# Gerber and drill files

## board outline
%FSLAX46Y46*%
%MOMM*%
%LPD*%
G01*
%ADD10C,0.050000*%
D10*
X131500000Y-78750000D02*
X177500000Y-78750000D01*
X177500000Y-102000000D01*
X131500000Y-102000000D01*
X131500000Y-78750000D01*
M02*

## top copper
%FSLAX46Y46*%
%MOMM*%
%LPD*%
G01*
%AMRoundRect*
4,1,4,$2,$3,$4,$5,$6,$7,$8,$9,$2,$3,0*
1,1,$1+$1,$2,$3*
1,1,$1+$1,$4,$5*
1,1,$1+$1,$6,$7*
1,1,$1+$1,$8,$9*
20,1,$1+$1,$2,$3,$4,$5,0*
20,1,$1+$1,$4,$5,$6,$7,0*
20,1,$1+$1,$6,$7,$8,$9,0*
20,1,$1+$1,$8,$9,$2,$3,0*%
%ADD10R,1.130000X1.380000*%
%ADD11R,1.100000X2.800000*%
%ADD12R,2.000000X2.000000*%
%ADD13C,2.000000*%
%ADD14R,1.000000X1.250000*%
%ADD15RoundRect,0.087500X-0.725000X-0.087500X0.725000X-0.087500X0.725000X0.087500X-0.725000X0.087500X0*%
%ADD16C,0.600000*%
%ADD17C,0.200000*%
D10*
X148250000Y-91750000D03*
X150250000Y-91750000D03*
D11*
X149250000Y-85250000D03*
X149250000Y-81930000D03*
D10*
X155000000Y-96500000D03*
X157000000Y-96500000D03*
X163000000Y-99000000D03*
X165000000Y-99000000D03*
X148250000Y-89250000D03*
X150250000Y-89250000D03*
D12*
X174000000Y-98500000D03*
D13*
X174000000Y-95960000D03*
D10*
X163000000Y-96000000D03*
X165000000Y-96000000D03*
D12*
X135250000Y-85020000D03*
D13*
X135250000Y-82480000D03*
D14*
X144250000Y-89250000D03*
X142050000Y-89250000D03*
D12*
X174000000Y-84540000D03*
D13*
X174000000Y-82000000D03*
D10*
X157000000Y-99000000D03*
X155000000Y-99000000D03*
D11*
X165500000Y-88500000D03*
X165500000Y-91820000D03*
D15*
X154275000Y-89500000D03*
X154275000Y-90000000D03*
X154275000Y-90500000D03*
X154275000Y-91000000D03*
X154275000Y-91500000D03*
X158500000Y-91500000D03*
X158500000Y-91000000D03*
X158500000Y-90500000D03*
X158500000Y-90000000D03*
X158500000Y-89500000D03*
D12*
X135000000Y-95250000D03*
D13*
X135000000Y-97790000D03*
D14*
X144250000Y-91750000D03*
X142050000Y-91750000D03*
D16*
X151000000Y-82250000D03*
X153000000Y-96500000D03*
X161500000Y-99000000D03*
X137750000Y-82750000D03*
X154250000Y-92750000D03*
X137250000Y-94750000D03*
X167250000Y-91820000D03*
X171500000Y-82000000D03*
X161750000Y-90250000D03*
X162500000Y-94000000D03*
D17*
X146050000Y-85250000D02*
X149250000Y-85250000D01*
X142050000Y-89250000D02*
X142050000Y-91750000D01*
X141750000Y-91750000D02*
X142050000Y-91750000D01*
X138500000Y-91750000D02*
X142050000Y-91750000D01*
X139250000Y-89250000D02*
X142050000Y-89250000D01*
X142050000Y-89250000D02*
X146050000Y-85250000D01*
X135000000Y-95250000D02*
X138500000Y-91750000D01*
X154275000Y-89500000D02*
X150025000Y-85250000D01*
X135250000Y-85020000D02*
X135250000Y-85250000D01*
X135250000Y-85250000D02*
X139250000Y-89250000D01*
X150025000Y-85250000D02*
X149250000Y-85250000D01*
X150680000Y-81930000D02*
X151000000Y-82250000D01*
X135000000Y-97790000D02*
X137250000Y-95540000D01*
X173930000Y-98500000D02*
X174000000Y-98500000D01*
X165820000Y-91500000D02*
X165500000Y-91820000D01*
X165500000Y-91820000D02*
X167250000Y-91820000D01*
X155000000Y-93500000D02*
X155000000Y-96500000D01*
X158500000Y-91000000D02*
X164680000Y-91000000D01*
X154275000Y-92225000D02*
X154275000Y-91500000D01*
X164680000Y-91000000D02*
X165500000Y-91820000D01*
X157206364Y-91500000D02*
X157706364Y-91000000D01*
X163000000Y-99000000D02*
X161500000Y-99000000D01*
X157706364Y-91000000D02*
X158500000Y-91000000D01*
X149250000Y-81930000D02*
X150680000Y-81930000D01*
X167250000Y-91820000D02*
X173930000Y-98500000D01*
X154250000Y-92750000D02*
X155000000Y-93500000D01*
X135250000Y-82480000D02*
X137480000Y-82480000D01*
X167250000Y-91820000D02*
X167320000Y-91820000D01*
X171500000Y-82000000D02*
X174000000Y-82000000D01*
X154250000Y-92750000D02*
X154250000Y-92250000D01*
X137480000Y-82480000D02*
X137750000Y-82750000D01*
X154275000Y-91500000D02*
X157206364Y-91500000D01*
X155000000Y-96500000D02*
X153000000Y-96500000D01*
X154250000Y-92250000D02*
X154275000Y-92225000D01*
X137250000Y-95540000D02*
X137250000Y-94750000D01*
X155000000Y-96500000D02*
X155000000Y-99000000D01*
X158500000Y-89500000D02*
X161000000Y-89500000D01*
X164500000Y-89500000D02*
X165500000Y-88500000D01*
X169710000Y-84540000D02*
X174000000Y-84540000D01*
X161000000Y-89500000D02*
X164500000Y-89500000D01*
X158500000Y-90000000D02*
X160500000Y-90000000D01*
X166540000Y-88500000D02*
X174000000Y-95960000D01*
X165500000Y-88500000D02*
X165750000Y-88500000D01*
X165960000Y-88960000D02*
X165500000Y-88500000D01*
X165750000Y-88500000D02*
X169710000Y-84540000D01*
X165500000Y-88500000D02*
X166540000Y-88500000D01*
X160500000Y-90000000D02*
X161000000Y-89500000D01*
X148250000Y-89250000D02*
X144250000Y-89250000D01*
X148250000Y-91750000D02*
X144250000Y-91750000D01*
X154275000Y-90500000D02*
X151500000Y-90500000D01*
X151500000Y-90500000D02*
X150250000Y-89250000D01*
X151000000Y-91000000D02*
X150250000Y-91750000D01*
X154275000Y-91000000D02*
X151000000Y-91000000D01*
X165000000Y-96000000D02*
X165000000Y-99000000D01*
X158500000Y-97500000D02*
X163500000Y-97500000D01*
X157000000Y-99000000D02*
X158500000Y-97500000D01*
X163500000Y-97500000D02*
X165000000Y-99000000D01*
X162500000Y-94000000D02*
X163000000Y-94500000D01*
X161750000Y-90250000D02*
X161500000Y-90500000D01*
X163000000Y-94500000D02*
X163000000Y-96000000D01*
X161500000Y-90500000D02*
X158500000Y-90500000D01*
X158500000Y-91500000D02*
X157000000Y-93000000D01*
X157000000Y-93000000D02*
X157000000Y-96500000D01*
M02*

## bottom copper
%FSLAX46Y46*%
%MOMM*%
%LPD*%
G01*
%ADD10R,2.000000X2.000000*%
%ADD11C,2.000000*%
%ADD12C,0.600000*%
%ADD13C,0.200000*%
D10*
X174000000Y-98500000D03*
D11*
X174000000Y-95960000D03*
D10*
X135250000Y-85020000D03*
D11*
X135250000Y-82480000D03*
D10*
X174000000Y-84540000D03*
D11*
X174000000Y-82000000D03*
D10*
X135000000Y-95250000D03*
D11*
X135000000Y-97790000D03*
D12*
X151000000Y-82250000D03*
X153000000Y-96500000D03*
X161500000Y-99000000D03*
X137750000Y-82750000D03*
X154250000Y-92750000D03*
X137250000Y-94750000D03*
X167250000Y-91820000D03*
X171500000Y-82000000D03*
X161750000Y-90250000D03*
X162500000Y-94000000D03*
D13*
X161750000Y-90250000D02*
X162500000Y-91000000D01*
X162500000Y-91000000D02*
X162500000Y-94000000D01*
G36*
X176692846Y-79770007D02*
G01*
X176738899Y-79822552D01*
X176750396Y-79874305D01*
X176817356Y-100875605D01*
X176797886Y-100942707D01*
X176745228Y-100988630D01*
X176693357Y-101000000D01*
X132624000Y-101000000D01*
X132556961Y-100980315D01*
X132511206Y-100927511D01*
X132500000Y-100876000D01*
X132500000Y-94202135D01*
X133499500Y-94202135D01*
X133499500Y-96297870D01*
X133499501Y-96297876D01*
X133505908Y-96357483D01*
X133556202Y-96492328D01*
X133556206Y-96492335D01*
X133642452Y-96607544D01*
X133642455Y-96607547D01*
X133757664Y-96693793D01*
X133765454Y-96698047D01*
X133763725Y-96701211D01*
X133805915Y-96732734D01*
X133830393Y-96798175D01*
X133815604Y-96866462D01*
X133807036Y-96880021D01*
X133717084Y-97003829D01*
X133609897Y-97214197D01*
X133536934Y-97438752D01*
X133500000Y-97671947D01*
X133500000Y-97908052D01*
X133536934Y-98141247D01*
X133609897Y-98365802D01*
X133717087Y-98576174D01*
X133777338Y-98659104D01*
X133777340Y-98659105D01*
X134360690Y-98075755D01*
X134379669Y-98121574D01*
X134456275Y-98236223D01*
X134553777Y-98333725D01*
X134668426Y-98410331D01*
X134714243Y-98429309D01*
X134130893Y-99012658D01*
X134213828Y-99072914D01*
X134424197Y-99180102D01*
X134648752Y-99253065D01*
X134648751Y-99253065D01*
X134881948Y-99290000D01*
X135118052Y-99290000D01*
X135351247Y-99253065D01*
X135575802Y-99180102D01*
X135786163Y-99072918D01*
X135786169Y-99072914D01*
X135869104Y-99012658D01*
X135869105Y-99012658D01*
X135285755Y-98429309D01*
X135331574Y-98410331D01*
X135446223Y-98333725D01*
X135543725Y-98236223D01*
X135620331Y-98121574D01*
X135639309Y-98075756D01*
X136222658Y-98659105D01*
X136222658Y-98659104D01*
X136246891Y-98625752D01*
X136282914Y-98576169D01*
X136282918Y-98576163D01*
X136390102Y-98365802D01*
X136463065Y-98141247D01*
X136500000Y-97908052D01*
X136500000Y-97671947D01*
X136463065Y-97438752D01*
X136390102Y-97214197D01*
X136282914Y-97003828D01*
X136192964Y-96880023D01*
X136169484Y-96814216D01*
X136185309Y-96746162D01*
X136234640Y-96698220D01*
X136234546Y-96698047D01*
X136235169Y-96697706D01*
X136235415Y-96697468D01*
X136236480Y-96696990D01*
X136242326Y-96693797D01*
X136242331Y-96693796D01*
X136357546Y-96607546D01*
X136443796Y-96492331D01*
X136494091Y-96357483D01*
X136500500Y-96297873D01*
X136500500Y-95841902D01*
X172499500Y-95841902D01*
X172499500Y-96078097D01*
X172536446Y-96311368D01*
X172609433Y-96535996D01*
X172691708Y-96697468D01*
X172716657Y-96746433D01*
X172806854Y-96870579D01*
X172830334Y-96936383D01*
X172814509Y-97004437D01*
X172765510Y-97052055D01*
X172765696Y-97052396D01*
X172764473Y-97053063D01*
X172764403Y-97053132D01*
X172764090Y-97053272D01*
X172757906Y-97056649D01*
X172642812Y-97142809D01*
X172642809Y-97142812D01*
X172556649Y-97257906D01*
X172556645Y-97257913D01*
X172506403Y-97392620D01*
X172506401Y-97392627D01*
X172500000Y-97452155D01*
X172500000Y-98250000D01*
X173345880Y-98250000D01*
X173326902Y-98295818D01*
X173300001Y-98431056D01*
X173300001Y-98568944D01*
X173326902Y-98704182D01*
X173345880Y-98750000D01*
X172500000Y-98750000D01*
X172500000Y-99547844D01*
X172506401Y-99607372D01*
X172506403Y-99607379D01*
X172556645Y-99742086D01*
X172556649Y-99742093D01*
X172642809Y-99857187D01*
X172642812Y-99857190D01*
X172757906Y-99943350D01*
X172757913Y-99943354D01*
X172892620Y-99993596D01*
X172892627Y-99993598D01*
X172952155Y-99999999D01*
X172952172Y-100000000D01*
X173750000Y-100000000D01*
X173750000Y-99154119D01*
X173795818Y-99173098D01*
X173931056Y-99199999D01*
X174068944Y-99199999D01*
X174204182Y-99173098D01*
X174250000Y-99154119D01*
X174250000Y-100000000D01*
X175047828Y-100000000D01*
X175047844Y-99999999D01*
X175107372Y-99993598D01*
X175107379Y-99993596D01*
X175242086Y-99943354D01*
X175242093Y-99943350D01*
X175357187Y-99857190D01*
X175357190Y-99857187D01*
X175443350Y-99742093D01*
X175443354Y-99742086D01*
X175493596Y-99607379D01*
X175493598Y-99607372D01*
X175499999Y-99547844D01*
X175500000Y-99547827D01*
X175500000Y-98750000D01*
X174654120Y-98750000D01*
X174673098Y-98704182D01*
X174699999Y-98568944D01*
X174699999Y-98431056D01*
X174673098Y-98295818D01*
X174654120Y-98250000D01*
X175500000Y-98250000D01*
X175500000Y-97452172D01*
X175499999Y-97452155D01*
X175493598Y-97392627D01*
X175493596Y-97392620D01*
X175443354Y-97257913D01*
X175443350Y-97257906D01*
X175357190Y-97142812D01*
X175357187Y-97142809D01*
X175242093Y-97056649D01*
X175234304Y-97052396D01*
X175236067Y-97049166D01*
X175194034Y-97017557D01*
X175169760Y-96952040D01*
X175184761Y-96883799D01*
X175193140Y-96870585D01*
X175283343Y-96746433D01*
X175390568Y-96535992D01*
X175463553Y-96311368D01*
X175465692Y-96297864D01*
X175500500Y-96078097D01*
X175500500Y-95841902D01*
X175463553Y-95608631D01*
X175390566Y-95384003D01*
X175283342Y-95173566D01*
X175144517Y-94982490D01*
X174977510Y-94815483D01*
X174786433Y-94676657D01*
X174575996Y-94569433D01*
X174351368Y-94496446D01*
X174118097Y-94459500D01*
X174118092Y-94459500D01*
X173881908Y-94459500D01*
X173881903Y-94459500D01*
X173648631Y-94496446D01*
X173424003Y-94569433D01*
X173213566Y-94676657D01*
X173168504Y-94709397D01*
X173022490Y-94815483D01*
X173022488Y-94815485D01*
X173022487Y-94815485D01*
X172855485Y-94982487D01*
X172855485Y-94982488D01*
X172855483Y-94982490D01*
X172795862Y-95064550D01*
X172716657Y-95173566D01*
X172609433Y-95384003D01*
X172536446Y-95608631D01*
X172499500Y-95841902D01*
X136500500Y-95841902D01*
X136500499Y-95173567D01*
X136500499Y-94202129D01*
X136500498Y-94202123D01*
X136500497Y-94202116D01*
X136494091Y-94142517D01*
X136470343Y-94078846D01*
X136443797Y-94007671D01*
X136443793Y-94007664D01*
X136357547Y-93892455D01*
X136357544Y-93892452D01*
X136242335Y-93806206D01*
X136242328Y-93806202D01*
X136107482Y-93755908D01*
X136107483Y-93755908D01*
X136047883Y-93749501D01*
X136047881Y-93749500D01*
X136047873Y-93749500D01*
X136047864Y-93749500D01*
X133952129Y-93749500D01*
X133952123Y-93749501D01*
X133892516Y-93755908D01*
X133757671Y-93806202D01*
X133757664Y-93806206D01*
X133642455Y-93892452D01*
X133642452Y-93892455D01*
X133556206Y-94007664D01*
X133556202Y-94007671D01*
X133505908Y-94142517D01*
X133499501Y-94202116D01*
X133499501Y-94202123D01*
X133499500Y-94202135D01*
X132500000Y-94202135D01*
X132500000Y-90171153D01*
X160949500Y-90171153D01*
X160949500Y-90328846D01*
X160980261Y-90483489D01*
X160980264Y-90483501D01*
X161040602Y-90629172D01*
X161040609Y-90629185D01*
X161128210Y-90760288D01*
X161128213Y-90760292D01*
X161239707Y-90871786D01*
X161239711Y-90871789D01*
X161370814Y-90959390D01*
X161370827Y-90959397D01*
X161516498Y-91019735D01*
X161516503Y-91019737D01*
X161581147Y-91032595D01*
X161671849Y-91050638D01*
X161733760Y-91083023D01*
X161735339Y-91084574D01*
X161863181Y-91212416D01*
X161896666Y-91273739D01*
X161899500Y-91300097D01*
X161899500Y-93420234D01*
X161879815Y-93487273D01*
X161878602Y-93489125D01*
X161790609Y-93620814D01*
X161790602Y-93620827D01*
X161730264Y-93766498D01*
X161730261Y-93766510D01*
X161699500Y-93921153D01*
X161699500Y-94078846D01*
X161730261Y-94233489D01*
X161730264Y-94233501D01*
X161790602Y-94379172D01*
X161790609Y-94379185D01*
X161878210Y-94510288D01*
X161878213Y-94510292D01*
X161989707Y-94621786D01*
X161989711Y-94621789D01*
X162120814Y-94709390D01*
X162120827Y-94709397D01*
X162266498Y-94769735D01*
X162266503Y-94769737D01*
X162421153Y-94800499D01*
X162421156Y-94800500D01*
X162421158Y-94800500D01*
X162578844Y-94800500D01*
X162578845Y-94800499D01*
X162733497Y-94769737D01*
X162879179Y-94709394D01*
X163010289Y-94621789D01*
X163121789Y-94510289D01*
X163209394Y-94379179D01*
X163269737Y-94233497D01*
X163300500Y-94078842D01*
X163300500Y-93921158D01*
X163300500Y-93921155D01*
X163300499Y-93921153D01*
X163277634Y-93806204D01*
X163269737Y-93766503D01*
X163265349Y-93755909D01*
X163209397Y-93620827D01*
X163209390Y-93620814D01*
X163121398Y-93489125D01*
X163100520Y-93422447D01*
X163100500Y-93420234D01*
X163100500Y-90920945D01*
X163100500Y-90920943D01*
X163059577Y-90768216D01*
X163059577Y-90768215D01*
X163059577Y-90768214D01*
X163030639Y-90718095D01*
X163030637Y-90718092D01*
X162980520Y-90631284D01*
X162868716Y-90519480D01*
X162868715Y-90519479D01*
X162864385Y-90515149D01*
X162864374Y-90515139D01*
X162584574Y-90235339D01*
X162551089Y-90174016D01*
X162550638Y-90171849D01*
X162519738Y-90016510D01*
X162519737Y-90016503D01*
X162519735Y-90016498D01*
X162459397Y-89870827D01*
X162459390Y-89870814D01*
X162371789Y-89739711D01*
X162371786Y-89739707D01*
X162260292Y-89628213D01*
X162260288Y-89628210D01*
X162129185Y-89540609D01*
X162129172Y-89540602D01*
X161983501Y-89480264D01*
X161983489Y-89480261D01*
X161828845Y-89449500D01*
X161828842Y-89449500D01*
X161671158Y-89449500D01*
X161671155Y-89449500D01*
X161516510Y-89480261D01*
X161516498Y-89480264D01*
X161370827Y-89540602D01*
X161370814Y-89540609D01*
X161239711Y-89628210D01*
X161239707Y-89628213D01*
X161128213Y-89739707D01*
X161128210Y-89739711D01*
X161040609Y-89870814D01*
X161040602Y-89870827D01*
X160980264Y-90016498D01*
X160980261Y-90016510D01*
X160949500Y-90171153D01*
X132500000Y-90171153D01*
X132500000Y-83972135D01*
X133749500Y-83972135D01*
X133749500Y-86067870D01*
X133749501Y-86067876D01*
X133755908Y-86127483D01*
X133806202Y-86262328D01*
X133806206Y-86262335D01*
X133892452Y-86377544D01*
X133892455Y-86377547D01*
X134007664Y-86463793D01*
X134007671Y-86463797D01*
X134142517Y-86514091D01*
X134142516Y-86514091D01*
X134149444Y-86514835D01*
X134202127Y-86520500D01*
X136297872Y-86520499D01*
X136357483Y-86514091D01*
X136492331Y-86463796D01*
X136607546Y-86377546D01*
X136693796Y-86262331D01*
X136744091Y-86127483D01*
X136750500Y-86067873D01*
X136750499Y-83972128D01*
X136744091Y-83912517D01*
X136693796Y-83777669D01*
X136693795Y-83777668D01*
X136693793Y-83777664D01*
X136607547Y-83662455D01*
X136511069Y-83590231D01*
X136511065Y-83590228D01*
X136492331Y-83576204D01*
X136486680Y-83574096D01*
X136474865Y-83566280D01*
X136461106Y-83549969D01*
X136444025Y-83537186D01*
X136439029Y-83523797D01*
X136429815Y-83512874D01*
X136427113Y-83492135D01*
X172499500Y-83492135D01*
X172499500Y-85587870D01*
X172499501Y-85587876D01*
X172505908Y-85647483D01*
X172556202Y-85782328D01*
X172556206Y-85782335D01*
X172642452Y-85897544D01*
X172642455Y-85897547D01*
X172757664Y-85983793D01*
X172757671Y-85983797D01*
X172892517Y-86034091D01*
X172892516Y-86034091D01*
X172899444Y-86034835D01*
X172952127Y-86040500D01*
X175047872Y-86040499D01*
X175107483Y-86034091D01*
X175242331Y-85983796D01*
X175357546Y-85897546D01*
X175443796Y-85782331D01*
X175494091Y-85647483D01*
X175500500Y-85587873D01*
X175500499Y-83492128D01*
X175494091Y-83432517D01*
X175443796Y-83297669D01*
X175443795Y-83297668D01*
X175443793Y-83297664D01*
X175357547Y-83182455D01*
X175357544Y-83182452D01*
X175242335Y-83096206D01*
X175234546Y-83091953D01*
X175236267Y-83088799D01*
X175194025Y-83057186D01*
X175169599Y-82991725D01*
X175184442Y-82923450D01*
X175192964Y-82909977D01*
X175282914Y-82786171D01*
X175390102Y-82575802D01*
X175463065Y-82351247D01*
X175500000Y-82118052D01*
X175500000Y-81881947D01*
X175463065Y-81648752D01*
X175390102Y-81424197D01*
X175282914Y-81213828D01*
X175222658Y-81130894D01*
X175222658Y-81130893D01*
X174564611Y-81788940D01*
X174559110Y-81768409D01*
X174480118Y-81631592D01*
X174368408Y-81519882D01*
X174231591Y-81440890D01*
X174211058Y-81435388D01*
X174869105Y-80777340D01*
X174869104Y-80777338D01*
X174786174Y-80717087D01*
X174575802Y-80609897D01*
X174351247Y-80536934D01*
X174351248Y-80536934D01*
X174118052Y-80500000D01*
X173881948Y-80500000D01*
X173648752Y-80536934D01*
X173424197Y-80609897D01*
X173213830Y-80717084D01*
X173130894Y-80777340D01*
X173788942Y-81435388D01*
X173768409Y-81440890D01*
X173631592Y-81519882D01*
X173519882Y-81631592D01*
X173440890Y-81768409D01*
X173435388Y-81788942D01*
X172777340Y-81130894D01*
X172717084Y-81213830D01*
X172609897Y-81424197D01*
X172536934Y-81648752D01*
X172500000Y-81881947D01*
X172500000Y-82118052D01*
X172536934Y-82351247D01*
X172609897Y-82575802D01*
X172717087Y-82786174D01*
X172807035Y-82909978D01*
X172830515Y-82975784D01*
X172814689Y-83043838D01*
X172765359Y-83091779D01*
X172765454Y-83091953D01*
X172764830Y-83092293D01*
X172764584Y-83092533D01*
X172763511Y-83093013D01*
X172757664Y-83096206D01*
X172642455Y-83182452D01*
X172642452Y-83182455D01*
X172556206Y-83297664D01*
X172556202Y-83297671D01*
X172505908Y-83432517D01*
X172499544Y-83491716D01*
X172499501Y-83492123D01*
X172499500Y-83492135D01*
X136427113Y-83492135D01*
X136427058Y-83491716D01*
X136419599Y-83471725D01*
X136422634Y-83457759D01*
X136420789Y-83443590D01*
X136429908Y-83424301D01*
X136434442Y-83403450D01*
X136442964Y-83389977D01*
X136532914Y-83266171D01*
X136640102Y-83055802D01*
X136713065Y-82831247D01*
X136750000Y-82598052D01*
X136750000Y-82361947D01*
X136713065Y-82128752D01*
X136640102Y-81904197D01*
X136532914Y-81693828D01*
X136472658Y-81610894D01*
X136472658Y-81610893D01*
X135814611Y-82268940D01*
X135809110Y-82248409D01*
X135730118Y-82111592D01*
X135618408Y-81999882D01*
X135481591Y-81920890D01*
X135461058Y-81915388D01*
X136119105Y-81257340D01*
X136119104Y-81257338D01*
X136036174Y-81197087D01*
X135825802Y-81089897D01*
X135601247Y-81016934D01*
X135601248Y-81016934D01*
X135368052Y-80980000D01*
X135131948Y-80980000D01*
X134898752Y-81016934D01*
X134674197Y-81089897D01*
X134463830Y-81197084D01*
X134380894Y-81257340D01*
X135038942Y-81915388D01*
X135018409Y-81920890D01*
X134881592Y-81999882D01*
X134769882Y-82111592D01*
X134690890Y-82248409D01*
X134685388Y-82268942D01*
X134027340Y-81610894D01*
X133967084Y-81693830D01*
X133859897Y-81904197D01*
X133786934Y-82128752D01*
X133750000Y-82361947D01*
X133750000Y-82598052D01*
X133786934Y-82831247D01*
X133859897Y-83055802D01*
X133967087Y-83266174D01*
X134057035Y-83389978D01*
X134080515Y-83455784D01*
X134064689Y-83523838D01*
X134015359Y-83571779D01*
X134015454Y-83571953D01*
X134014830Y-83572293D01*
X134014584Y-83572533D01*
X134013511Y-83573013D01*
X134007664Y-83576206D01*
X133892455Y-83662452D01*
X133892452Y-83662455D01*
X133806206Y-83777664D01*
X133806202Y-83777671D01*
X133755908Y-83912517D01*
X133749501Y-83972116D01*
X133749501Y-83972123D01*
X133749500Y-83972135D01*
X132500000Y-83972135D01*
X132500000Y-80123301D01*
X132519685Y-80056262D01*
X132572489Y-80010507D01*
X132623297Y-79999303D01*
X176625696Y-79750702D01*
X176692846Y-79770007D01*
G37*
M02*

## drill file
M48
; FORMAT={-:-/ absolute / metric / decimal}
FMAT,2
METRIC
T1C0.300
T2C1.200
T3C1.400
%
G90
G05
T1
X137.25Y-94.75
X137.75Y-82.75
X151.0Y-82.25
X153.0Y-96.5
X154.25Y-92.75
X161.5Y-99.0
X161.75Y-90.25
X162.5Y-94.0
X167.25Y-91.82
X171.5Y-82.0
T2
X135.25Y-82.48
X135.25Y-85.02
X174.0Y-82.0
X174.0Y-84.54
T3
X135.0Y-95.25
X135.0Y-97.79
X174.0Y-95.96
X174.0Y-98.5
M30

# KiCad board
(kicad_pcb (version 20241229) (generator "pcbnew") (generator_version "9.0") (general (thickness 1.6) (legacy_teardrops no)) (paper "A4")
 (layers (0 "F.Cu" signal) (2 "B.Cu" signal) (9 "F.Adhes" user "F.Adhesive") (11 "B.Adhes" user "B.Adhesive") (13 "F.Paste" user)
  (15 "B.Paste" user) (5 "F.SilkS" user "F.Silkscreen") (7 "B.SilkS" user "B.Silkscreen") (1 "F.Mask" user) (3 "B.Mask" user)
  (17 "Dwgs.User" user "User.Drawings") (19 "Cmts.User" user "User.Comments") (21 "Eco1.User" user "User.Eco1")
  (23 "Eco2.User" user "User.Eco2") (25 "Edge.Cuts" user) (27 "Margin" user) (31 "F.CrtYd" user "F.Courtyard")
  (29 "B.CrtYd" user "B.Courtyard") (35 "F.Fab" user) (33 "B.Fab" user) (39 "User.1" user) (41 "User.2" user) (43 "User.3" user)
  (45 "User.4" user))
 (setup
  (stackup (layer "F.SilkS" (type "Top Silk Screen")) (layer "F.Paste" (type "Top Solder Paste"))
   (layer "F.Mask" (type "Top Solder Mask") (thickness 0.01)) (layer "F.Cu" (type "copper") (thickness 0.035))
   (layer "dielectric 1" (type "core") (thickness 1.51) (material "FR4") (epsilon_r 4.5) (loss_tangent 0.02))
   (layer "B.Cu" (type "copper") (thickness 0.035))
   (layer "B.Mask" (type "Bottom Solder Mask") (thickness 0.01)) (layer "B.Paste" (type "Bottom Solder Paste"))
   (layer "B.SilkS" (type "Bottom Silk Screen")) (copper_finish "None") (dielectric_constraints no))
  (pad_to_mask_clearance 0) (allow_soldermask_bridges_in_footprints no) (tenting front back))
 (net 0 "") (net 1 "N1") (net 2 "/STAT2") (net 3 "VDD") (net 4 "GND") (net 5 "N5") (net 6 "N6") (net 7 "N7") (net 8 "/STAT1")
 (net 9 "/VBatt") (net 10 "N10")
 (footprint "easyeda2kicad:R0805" (layer "F.Cu") (at 149.25 91.75)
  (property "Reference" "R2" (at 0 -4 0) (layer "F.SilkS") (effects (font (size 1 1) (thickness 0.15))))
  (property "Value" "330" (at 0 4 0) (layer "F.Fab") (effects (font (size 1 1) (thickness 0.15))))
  (pad "1" smd rect (at -1 0) (size 1.13 1.38) (layers "F.Cu" "F.Mask" "F.Paste") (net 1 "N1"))
  (pad "2" smd rect (at 1 0) (size 1.13 1.38) (layers "F.Cu" "F.Mask" "F.Paste") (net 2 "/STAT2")))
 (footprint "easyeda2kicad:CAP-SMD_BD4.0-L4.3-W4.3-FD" (layer "F.Cu") (at 149.25 83.59 90)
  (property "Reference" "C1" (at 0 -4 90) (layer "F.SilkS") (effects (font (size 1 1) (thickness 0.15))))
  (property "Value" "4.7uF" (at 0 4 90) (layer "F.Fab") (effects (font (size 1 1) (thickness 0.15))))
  (pad "1" smd rect (at -1.66 0 90) (size 2.8 1.1) (layers "F.Cu" "F.Mask" "F.Paste") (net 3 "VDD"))
  (pad "2" smd rect (at 1.66 0 90) (size 2.8 1.1) (layers "F.Cu" "F.Mask" "F.Paste") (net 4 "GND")))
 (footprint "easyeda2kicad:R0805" (layer "F.Cu") (at 156 96.5)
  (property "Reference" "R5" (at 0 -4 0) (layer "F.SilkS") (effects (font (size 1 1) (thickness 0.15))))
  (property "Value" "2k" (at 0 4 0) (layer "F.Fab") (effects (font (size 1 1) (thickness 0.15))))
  (pad "1" smd rect (at -1 0) (size 1.13 1.38) (layers "F.Cu" "F.Mask" "F.Paste") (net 4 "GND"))
  (pad "2" smd rect (at 1 0) (size 1.13 1.38) (layers "F.Cu" "F.Mask" "F.Paste") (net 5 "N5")))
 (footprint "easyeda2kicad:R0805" (layer "F.Cu") (at 164 99)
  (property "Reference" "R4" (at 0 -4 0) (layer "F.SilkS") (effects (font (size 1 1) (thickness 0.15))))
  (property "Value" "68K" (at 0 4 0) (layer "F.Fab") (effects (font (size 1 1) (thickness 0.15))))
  (pad "1" smd rect (at -1 0) (size 1.13 1.38) (layers "F.Cu" "F.Mask" "F.Paste") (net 4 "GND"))
  (pad "2" smd rect (at 1 0) (size 1.13 1.38) (layers "F.Cu" "F.Mask" "F.Paste") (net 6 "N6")))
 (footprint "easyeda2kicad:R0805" (layer "F.Cu") (at 149.25 89.25)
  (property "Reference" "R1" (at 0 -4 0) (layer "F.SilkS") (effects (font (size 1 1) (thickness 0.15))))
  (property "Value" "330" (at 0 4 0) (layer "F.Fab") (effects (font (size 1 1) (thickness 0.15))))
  (pad "1" smd rect (at -1 0) (size 1.13 1.38) (layers "F.Cu" "F.Mask" "F.Paste") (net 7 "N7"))
  (pad "2" smd rect (at 1 0) (size 1.13 1.38) (layers "F.Cu" "F.Mask" "F.Paste") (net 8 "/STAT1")))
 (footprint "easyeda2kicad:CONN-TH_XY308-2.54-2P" (layer "F.Cu") (at 174 97.23 90)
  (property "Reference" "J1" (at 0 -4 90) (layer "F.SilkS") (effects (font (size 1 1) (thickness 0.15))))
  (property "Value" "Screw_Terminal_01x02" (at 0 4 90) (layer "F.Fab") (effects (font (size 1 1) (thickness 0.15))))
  (pad "1" thru_hole rect (at -1.27 0 90) (size 2 2) (drill 1.399997) (layers "*.Cu" "*.Mask") (remove_unused_layers no) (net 4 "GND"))
  (pad "2" thru_hole circle (at 1.27 0 90) (size 2 2) (drill 1.399997) (layers "*.Cu" "*.Mask") (remove_unused_layers no) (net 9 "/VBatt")))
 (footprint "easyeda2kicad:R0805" (layer "F.Cu") (at 164 96)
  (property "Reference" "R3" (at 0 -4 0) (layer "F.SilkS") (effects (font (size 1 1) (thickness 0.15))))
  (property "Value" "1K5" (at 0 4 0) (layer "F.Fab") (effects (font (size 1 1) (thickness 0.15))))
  (pad "1" smd rect (at -1 0) (size 1.13 1.38) (layers "F.Cu" "F.Mask" "F.Paste") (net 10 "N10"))
  (pad "2" smd rect (at 1 0) (size 1.13 1.38) (layers "F.Cu" "F.Mask" "F.Paste") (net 6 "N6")))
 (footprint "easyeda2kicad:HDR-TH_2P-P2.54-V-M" (layer "F.Cu") (at 135.25 83.75 90)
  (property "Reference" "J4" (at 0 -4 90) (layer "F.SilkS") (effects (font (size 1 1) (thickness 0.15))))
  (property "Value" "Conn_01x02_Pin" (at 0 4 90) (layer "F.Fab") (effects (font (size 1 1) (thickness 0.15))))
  (pad "1" thru_hole rect (at -1.27 0 90) (size 2 2) (drill 1.199998) (layers "*.Cu" "*.Mask") (remove_unused_layers no) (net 3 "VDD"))
  (pad "2" thru_hole circle (at 1.27 0 90) (size 2 2) (drill 1.199998) (layers "*.Cu" "*.Mask") (remove_unused_layers no) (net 4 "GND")))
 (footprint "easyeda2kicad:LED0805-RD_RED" (layer "F.Cu") (at 143.15 89.25 180)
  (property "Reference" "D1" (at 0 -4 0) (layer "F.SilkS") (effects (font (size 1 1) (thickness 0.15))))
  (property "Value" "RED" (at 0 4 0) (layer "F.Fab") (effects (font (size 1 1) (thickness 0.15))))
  (pad "1" smd rect (at -1.1 0) (size 1 1.25) (layers "F.Cu" "F.Mask" "F.Paste") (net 7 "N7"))
  (pad "2" smd rect (at 1.1 0) (size 1 1.25) (layers "F.Cu" "F.Mask" "F.Paste") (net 3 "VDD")))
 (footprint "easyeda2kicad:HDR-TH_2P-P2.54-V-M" (layer "F.Cu") (at 174 83.27 90)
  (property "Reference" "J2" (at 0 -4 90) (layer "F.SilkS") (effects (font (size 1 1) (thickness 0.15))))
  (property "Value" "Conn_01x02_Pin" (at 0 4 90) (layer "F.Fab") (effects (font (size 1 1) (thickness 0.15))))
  (pad "1" thru_hole rect (at -1.27 0 90) (size 2 2) (drill 1.199998) (layers "*.Cu" "*.Mask") (remove_unused_layers no) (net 9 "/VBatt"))
  (pad "2" thru_hole circle (at 1.27 0 90) (size 2 2) (drill 1.199998) (layers "*.Cu" "*.Mask") (remove_unused_layers no) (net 4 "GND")))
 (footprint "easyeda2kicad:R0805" (layer "F.Cu") (at 156 99 180)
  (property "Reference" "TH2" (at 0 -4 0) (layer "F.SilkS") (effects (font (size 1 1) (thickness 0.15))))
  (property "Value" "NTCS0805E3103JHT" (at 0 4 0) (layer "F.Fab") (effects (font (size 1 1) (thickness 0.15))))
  (pad "1" smd rect (at -1 0 180) (size 1.13 1.38) (layers "F.Cu" "F.Mask" "F.Paste") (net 6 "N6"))
  (pad "2" smd rect (at 1 0 180) (size 1.13 1.38) (layers "F.Cu" "F.Mask" "F.Paste") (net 4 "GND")))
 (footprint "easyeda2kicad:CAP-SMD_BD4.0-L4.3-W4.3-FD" (layer "F.Cu") (at 165.5 90.16 -90)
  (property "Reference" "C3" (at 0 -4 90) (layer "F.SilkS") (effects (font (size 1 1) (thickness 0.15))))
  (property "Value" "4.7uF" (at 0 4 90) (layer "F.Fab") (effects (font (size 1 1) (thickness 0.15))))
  (pad "1" smd rect (at -1.66 0 270) (size 2.8 1.1) (layers "F.Cu" "F.Mask" "F.Paste") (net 9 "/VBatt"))
  (pad "2" smd rect (at 1.66 0 270) (size 2.8 1.1) (layers "F.Cu" "F.Mask" "F.Paste") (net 4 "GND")))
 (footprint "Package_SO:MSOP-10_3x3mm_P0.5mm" (layer "F.Cu") (at 156.3875 90.5)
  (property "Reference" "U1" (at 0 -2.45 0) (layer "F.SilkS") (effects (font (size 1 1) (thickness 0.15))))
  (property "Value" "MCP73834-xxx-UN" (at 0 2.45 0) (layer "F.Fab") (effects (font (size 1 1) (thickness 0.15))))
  (pad "1" smd roundrect (at -2.1125 -1) (size 1.625 0.35) (layers "F.Cu" "F.Mask" "F.Paste") (roundrect_rratio 0.25) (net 3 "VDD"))
  (pad "2" smd roundrect (at -2.1125 -0.5) (size 1.625 0.35) (layers "F.Cu" "F.Mask" "F.Paste") (roundrect_rratio 0.25) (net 3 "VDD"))
  (pad "3" smd roundrect (at -2.1125 0) (size 1.625 0.35) (layers "F.Cu" "F.Mask" "F.Paste") (roundrect_rratio 0.25) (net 8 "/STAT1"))
  (pad "4" smd roundrect (at -2.1125 0.5) (size 1.625 0.35) (layers "F.Cu" "F.Mask" "F.Paste") (roundrect_rratio 0.25) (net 2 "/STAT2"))
  (pad "5" smd roundrect (at -2.1125 1) (size 1.625 0.35) (layers "F.Cu" "F.Mask" "F.Paste") (roundrect_rratio 0.25) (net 4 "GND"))
  (pad "6" smd roundrect (at 2.1125 1) (size 1.625 0.35) (layers "F.Cu" "F.Mask" "F.Paste") (roundrect_rratio 0.25) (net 5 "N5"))
  (pad "7" smd roundrect (at 2.1125 0.5) (size 1.625 0.35) (layers "F.Cu" "F.Mask" "F.Paste") (roundrect_rratio 0.25) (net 4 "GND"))
  (pad "8" smd roundrect (at 2.1125 0) (size 1.625 0.35) (layers "F.Cu" "F.Mask" "F.Paste") (roundrect_rratio 0.25) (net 10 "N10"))
  (pad "9" smd roundrect (at 2.1125 -0.5) (size 1.625 0.35) (layers "F.Cu" "F.Mask" "F.Paste") (roundrect_rratio 0.25) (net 9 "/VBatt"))
  (pad "10" smd roundrect (at 2.1125 -1) (size 1.625 0.35) (layers "F.Cu" "F.Mask" "F.Paste") (roundrect_rratio 0.25) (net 9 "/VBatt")))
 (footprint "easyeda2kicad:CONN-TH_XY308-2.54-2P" (layer "F.Cu") (at 135 96.52 -90)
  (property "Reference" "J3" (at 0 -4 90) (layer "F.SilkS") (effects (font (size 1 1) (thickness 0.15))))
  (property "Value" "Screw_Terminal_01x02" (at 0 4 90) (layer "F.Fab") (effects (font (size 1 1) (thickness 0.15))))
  (pad "1" thru_hole rect (at -1.27 0 270) (size 2 2) (drill 1.399997) (layers "*.Cu" "*.Mask") (remove_unused_layers no) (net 3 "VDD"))
  (pad "2" thru_hole circle (at 1.27 0 270) (size 2 2) (drill 1.399997) (layers "*.Cu" "*.Mask") (remove_unused_layers no) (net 4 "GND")))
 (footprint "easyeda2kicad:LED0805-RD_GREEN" (layer "F.Cu") (at 143.15 91.75 180)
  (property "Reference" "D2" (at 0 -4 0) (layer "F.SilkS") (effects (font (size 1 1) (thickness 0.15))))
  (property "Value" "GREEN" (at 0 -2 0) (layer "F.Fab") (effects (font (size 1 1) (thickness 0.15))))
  (pad "1" smd rect (at -1.1 0) (size 1 1.25) (layers "F.Cu" "F.Mask" "F.Paste") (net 1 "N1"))
  (pad "2" smd rect (at 1.1 0) (size 1 1.25) (layers "F.Cu" "F.Mask" "F.Paste") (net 3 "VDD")))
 (gr_rect (start 131.5 78.75) (end 177.5 102) (stroke (width 0.05) (type default)) (fill no) (layer "Edge.Cuts"))
 (segment (start 146.05 85.25) (end 149.25 85.25) (width 0.2) (layer "F.Cu") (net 3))
 (segment (start 142.05 89.25) (end 142.05 91.75) (width 0.2) (layer "F.Cu") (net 3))
 (segment (start 141.75 91.75) (end 142.05 91.75) (width 0.2) (layer "F.Cu") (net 3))
 (segment (start 138.5 91.75) (end 142.05 91.75) (width 0.2) (layer "F.Cu") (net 3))
 (segment (start 139.25 89.25) (end 142.05 89.25) (width 0.2) (layer "F.Cu") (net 3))
 (segment (start 142.05 89.25) (end 146.05 85.25) (width 0.2) (layer "F.Cu") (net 3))
 (segment (start 135 95.25) (end 138.5 91.75) (width 0.2) (layer "F.Cu") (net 3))
 (segment (start 154.275 89.5) (end 150.025 85.25) (width 0.2) (layer "F.Cu") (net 3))
 (segment (start 135.25 85.02) (end 135.25 85.25) (width 0.2) (layer "F.Cu") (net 3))
 (segment (start 135.25 85.25) (end 139.25 89.25) (width 0.2) (layer "F.Cu") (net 3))
 (segment (start 150.025 85.25) (end 149.25 85.25) (width 0.2) (layer "F.Cu") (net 3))
 (segment (start 150.68 81.93) (end 151 82.25) (width 0.2) (layer "F.Cu") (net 4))
 (segment (start 135 97.79) (end 137.25 95.54) (width 0.2) (layer "F.Cu") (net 4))
 (segment (start 173.93 98.5) (end 174 98.5) (width 0.2) (layer "F.Cu") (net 4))
 (segment (start 165.82 91.5) (end 165.5 91.82) (width 0.2) (layer "F.Cu") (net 4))
 (segment (start 165.5 91.82) (end 167.25 91.82) (width 0.2) (layer "F.Cu") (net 4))
 (segment (start 155 93.5) (end 155 96.5) (width 0.2) (layer "F.Cu") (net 4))
 (segment (start 158.5 91) (end 164.68 91) (width 0.2) (layer "F.Cu") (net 4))
 (segment (start 154.275 92.225) (end 154.275 91.5) (width 0.2) (layer "F.Cu") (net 4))
 (segment (start 164.68 91) (end 165.5 91.82) (width 0.2) (layer "F.Cu") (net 4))
 (segment (start 157.206364 91.5) (end 157.706364 91) (width 0.2) (layer "F.Cu") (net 4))
 (segment (start 163 99) (end 161.5 99) (width 0.2) (layer "F.Cu") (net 4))
 (segment (start 157.706364 91) (end 158.5 91) (width 0.2) (layer "F.Cu") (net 4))
 (segment (start 149.25 81.93) (end 150.68 81.93) (width 0.2) (layer "F.Cu") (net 4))
 (segment (start 167.25 91.82) (end 173.93 98.5) (width 0.2) (layer "F.Cu") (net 4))
 (segment (start 154.25 92.75) (end 155 93.5) (width 0.2) (layer "F.Cu") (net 4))
 (segment (start 135.25 82.48) (end 137.48 82.48) (width 0.2) (layer "F.Cu") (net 4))
 (segment (start 167.25 91.82) (end 167.32 91.82) (width 0.2) (layer "F.Cu") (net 4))
 (segment (start 171.5 82) (end 174 82) (width 0.2) (layer "F.Cu") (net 4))
 (segment (start 154.25 92.75) (end 154.25 92.25) (width 0.2) (layer "F.Cu") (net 4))
 (segment (start 137.48 82.48) (end 137.75 82.75) (width 0.2) (layer "F.Cu") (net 4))
 (segment (start 154.275 91.5) (end 157.206364 91.5) (width 0.2) (layer "F.Cu") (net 4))
 (segment (start 155 96.5) (end 153 96.5) (width 0.2) (layer "F.Cu") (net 4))
 (segment (start 154.25 92.25) (end 154.275 92.225) (width 0.2) (layer "F.Cu") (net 4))
 (segment (start 137.25 95.54) (end 137.25 94.75) (width 0.2) (layer "F.Cu") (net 4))
 (segment (start 155 96.5) (end 155 99) (width 0.2) (layer "F.Cu") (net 4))
 (via (at 151 82.25) (size 0.6) (drill 0.3) (layers "F.Cu" "B.Cu") (free yes) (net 4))
 (via (at 153 96.5) (size 0.6) (drill 0.3) (layers "F.Cu" "B.Cu") (free yes) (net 4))
 (via (at 161.5 99) (size 0.6) (drill 0.3) (layers "F.Cu" "B.Cu") (free yes) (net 4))
 (via (at 137.75 82.75) (size 0.6) (drill 0.3) (layers "F.Cu" "B.Cu") (free yes) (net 4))
 (via (at 154.25 92.75) (size 0.6) (drill 0.3) (layers "F.Cu" "B.Cu") (free yes) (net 4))
 (via (at 137.25 94.75) (size 0.6) (drill 0.3) (layers "F.Cu" "B.Cu") (free yes) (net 4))
 (via (at 167.25 91.82) (size 0.6) (drill 0.3) (layers "F.Cu" "B.Cu") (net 4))
 (via (at 171.5 82) (size 0.6) (drill 0.3) (layers "F.Cu" "B.Cu") (free yes) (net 4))
 (segment (start 158.5 89.5) (end 161 89.5) (width 0.2) (layer "F.Cu") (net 9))
 (segment (start 164.5 89.5) (end 165.5 88.5) (width 0.2) (layer "F.Cu") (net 9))
 (segment (start 169.71 84.54) (end 174 84.54) (width 0.2) (layer "F.Cu") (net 9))
 (segment (start 161 89.5) (end 164.5 89.5) (width 0.2) (layer "F.Cu") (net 9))
 (segment (start 158.5 90) (end 160.5 90) (width 0.2) (layer "F.Cu") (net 9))
 (segment (start 166.54 88.5) (end 174 95.96) (width 0.2) (layer "F.Cu") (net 9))
 (segment (start 165.5 88.5) (end 165.75 88.5) (width 0.2) (layer "F.Cu") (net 9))
 (segment (start 165.96 88.96) (end 165.5 88.5) (width 0.2) (layer "F.Cu") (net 9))
 (segment (start 165.75 88.5) (end 169.71 84.54) (width 0.2) (layer "F.Cu") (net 9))
 (segment (start 165.5 88.5) (end 166.54 88.5) (width 0.2) (layer "F.Cu") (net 9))
 (segment (start 160.5 90) (end 161 89.5) (width 0.2) (layer "F.Cu") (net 9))
 (segment (start 148.25 89.25) (end 144.25 89.25) (width 0.2) (layer "F.Cu") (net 7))
 (segment (start 148.25 91.75) (end 144.25 91.75) (width 0.2) (layer "F.Cu") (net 1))
 (segment (start 154.275 90.5) (end 151.5 90.5) (width 0.2) (layer "F.Cu") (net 8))
 (segment (start 151.5 90.5) (end 150.25 89.25) (width 0.2) (layer "F.Cu") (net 8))
 (segment (start 151 91) (end 150.25 91.75) (width 0.2) (layer "F.Cu") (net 2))
 (segment (start 154.275 91) (end 151 91) (width 0.2) (layer "F.Cu") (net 2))
 (segment (start 165 96) (end 165 99) (width 0.2) (layer "F.Cu") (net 6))
 (segment (start 158.5 97.5) (end 163.5 97.5) (width 0.2) (layer "F.Cu") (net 6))
 (segment (start 157 99) (end 158.5 97.5) (width 0.2) (layer "F.Cu") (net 6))
 (segment (start 163.5 97.5) (end 165 99) (width 0.2) (layer "F.Cu") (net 6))
 (segment (start 162.5 94) (end 163 94.5) (width 0.2) (layer "F.Cu") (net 10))
 (segment (start 161.75 90.25) (end 161.5 90.5) (width 0.2) (layer "F.Cu") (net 10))
 (segment (start 163 94.5) (end 163 96) (width 0.2) (layer "F.Cu") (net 10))
 (segment (start 161.5 90.5) (end 158.5 90.5) (width 0.2) (layer "F.Cu") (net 10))
 (via (at 161.75 90.25) (size 0.6) (drill 0.3) (layers "F.Cu" "B.Cu") (free yes) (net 10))
 (via (at 162.5 94) (size 0.6) (drill 0.3) (layers "F.Cu" "B.Cu") (free yes) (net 10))
 (segment (start 161.75 90.25) (end 162.5 91) (width 0.2) (layer "B.Cu") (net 10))
 (segment (start 162.5 91) (end 162.5 94) (width 0.2) (layer "B.Cu") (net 10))
 (segment (start 158.5 91.5) (end 157 93) (width 0.2) (layer "F.Cu") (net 5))
 (segment (start 157 93) (end 157 96.5) (width 0.2) (layer "F.Cu") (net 5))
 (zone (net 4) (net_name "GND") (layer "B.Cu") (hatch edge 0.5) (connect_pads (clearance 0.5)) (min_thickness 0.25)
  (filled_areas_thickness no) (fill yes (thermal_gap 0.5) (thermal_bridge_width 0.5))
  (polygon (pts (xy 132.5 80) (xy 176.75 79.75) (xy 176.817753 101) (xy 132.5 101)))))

